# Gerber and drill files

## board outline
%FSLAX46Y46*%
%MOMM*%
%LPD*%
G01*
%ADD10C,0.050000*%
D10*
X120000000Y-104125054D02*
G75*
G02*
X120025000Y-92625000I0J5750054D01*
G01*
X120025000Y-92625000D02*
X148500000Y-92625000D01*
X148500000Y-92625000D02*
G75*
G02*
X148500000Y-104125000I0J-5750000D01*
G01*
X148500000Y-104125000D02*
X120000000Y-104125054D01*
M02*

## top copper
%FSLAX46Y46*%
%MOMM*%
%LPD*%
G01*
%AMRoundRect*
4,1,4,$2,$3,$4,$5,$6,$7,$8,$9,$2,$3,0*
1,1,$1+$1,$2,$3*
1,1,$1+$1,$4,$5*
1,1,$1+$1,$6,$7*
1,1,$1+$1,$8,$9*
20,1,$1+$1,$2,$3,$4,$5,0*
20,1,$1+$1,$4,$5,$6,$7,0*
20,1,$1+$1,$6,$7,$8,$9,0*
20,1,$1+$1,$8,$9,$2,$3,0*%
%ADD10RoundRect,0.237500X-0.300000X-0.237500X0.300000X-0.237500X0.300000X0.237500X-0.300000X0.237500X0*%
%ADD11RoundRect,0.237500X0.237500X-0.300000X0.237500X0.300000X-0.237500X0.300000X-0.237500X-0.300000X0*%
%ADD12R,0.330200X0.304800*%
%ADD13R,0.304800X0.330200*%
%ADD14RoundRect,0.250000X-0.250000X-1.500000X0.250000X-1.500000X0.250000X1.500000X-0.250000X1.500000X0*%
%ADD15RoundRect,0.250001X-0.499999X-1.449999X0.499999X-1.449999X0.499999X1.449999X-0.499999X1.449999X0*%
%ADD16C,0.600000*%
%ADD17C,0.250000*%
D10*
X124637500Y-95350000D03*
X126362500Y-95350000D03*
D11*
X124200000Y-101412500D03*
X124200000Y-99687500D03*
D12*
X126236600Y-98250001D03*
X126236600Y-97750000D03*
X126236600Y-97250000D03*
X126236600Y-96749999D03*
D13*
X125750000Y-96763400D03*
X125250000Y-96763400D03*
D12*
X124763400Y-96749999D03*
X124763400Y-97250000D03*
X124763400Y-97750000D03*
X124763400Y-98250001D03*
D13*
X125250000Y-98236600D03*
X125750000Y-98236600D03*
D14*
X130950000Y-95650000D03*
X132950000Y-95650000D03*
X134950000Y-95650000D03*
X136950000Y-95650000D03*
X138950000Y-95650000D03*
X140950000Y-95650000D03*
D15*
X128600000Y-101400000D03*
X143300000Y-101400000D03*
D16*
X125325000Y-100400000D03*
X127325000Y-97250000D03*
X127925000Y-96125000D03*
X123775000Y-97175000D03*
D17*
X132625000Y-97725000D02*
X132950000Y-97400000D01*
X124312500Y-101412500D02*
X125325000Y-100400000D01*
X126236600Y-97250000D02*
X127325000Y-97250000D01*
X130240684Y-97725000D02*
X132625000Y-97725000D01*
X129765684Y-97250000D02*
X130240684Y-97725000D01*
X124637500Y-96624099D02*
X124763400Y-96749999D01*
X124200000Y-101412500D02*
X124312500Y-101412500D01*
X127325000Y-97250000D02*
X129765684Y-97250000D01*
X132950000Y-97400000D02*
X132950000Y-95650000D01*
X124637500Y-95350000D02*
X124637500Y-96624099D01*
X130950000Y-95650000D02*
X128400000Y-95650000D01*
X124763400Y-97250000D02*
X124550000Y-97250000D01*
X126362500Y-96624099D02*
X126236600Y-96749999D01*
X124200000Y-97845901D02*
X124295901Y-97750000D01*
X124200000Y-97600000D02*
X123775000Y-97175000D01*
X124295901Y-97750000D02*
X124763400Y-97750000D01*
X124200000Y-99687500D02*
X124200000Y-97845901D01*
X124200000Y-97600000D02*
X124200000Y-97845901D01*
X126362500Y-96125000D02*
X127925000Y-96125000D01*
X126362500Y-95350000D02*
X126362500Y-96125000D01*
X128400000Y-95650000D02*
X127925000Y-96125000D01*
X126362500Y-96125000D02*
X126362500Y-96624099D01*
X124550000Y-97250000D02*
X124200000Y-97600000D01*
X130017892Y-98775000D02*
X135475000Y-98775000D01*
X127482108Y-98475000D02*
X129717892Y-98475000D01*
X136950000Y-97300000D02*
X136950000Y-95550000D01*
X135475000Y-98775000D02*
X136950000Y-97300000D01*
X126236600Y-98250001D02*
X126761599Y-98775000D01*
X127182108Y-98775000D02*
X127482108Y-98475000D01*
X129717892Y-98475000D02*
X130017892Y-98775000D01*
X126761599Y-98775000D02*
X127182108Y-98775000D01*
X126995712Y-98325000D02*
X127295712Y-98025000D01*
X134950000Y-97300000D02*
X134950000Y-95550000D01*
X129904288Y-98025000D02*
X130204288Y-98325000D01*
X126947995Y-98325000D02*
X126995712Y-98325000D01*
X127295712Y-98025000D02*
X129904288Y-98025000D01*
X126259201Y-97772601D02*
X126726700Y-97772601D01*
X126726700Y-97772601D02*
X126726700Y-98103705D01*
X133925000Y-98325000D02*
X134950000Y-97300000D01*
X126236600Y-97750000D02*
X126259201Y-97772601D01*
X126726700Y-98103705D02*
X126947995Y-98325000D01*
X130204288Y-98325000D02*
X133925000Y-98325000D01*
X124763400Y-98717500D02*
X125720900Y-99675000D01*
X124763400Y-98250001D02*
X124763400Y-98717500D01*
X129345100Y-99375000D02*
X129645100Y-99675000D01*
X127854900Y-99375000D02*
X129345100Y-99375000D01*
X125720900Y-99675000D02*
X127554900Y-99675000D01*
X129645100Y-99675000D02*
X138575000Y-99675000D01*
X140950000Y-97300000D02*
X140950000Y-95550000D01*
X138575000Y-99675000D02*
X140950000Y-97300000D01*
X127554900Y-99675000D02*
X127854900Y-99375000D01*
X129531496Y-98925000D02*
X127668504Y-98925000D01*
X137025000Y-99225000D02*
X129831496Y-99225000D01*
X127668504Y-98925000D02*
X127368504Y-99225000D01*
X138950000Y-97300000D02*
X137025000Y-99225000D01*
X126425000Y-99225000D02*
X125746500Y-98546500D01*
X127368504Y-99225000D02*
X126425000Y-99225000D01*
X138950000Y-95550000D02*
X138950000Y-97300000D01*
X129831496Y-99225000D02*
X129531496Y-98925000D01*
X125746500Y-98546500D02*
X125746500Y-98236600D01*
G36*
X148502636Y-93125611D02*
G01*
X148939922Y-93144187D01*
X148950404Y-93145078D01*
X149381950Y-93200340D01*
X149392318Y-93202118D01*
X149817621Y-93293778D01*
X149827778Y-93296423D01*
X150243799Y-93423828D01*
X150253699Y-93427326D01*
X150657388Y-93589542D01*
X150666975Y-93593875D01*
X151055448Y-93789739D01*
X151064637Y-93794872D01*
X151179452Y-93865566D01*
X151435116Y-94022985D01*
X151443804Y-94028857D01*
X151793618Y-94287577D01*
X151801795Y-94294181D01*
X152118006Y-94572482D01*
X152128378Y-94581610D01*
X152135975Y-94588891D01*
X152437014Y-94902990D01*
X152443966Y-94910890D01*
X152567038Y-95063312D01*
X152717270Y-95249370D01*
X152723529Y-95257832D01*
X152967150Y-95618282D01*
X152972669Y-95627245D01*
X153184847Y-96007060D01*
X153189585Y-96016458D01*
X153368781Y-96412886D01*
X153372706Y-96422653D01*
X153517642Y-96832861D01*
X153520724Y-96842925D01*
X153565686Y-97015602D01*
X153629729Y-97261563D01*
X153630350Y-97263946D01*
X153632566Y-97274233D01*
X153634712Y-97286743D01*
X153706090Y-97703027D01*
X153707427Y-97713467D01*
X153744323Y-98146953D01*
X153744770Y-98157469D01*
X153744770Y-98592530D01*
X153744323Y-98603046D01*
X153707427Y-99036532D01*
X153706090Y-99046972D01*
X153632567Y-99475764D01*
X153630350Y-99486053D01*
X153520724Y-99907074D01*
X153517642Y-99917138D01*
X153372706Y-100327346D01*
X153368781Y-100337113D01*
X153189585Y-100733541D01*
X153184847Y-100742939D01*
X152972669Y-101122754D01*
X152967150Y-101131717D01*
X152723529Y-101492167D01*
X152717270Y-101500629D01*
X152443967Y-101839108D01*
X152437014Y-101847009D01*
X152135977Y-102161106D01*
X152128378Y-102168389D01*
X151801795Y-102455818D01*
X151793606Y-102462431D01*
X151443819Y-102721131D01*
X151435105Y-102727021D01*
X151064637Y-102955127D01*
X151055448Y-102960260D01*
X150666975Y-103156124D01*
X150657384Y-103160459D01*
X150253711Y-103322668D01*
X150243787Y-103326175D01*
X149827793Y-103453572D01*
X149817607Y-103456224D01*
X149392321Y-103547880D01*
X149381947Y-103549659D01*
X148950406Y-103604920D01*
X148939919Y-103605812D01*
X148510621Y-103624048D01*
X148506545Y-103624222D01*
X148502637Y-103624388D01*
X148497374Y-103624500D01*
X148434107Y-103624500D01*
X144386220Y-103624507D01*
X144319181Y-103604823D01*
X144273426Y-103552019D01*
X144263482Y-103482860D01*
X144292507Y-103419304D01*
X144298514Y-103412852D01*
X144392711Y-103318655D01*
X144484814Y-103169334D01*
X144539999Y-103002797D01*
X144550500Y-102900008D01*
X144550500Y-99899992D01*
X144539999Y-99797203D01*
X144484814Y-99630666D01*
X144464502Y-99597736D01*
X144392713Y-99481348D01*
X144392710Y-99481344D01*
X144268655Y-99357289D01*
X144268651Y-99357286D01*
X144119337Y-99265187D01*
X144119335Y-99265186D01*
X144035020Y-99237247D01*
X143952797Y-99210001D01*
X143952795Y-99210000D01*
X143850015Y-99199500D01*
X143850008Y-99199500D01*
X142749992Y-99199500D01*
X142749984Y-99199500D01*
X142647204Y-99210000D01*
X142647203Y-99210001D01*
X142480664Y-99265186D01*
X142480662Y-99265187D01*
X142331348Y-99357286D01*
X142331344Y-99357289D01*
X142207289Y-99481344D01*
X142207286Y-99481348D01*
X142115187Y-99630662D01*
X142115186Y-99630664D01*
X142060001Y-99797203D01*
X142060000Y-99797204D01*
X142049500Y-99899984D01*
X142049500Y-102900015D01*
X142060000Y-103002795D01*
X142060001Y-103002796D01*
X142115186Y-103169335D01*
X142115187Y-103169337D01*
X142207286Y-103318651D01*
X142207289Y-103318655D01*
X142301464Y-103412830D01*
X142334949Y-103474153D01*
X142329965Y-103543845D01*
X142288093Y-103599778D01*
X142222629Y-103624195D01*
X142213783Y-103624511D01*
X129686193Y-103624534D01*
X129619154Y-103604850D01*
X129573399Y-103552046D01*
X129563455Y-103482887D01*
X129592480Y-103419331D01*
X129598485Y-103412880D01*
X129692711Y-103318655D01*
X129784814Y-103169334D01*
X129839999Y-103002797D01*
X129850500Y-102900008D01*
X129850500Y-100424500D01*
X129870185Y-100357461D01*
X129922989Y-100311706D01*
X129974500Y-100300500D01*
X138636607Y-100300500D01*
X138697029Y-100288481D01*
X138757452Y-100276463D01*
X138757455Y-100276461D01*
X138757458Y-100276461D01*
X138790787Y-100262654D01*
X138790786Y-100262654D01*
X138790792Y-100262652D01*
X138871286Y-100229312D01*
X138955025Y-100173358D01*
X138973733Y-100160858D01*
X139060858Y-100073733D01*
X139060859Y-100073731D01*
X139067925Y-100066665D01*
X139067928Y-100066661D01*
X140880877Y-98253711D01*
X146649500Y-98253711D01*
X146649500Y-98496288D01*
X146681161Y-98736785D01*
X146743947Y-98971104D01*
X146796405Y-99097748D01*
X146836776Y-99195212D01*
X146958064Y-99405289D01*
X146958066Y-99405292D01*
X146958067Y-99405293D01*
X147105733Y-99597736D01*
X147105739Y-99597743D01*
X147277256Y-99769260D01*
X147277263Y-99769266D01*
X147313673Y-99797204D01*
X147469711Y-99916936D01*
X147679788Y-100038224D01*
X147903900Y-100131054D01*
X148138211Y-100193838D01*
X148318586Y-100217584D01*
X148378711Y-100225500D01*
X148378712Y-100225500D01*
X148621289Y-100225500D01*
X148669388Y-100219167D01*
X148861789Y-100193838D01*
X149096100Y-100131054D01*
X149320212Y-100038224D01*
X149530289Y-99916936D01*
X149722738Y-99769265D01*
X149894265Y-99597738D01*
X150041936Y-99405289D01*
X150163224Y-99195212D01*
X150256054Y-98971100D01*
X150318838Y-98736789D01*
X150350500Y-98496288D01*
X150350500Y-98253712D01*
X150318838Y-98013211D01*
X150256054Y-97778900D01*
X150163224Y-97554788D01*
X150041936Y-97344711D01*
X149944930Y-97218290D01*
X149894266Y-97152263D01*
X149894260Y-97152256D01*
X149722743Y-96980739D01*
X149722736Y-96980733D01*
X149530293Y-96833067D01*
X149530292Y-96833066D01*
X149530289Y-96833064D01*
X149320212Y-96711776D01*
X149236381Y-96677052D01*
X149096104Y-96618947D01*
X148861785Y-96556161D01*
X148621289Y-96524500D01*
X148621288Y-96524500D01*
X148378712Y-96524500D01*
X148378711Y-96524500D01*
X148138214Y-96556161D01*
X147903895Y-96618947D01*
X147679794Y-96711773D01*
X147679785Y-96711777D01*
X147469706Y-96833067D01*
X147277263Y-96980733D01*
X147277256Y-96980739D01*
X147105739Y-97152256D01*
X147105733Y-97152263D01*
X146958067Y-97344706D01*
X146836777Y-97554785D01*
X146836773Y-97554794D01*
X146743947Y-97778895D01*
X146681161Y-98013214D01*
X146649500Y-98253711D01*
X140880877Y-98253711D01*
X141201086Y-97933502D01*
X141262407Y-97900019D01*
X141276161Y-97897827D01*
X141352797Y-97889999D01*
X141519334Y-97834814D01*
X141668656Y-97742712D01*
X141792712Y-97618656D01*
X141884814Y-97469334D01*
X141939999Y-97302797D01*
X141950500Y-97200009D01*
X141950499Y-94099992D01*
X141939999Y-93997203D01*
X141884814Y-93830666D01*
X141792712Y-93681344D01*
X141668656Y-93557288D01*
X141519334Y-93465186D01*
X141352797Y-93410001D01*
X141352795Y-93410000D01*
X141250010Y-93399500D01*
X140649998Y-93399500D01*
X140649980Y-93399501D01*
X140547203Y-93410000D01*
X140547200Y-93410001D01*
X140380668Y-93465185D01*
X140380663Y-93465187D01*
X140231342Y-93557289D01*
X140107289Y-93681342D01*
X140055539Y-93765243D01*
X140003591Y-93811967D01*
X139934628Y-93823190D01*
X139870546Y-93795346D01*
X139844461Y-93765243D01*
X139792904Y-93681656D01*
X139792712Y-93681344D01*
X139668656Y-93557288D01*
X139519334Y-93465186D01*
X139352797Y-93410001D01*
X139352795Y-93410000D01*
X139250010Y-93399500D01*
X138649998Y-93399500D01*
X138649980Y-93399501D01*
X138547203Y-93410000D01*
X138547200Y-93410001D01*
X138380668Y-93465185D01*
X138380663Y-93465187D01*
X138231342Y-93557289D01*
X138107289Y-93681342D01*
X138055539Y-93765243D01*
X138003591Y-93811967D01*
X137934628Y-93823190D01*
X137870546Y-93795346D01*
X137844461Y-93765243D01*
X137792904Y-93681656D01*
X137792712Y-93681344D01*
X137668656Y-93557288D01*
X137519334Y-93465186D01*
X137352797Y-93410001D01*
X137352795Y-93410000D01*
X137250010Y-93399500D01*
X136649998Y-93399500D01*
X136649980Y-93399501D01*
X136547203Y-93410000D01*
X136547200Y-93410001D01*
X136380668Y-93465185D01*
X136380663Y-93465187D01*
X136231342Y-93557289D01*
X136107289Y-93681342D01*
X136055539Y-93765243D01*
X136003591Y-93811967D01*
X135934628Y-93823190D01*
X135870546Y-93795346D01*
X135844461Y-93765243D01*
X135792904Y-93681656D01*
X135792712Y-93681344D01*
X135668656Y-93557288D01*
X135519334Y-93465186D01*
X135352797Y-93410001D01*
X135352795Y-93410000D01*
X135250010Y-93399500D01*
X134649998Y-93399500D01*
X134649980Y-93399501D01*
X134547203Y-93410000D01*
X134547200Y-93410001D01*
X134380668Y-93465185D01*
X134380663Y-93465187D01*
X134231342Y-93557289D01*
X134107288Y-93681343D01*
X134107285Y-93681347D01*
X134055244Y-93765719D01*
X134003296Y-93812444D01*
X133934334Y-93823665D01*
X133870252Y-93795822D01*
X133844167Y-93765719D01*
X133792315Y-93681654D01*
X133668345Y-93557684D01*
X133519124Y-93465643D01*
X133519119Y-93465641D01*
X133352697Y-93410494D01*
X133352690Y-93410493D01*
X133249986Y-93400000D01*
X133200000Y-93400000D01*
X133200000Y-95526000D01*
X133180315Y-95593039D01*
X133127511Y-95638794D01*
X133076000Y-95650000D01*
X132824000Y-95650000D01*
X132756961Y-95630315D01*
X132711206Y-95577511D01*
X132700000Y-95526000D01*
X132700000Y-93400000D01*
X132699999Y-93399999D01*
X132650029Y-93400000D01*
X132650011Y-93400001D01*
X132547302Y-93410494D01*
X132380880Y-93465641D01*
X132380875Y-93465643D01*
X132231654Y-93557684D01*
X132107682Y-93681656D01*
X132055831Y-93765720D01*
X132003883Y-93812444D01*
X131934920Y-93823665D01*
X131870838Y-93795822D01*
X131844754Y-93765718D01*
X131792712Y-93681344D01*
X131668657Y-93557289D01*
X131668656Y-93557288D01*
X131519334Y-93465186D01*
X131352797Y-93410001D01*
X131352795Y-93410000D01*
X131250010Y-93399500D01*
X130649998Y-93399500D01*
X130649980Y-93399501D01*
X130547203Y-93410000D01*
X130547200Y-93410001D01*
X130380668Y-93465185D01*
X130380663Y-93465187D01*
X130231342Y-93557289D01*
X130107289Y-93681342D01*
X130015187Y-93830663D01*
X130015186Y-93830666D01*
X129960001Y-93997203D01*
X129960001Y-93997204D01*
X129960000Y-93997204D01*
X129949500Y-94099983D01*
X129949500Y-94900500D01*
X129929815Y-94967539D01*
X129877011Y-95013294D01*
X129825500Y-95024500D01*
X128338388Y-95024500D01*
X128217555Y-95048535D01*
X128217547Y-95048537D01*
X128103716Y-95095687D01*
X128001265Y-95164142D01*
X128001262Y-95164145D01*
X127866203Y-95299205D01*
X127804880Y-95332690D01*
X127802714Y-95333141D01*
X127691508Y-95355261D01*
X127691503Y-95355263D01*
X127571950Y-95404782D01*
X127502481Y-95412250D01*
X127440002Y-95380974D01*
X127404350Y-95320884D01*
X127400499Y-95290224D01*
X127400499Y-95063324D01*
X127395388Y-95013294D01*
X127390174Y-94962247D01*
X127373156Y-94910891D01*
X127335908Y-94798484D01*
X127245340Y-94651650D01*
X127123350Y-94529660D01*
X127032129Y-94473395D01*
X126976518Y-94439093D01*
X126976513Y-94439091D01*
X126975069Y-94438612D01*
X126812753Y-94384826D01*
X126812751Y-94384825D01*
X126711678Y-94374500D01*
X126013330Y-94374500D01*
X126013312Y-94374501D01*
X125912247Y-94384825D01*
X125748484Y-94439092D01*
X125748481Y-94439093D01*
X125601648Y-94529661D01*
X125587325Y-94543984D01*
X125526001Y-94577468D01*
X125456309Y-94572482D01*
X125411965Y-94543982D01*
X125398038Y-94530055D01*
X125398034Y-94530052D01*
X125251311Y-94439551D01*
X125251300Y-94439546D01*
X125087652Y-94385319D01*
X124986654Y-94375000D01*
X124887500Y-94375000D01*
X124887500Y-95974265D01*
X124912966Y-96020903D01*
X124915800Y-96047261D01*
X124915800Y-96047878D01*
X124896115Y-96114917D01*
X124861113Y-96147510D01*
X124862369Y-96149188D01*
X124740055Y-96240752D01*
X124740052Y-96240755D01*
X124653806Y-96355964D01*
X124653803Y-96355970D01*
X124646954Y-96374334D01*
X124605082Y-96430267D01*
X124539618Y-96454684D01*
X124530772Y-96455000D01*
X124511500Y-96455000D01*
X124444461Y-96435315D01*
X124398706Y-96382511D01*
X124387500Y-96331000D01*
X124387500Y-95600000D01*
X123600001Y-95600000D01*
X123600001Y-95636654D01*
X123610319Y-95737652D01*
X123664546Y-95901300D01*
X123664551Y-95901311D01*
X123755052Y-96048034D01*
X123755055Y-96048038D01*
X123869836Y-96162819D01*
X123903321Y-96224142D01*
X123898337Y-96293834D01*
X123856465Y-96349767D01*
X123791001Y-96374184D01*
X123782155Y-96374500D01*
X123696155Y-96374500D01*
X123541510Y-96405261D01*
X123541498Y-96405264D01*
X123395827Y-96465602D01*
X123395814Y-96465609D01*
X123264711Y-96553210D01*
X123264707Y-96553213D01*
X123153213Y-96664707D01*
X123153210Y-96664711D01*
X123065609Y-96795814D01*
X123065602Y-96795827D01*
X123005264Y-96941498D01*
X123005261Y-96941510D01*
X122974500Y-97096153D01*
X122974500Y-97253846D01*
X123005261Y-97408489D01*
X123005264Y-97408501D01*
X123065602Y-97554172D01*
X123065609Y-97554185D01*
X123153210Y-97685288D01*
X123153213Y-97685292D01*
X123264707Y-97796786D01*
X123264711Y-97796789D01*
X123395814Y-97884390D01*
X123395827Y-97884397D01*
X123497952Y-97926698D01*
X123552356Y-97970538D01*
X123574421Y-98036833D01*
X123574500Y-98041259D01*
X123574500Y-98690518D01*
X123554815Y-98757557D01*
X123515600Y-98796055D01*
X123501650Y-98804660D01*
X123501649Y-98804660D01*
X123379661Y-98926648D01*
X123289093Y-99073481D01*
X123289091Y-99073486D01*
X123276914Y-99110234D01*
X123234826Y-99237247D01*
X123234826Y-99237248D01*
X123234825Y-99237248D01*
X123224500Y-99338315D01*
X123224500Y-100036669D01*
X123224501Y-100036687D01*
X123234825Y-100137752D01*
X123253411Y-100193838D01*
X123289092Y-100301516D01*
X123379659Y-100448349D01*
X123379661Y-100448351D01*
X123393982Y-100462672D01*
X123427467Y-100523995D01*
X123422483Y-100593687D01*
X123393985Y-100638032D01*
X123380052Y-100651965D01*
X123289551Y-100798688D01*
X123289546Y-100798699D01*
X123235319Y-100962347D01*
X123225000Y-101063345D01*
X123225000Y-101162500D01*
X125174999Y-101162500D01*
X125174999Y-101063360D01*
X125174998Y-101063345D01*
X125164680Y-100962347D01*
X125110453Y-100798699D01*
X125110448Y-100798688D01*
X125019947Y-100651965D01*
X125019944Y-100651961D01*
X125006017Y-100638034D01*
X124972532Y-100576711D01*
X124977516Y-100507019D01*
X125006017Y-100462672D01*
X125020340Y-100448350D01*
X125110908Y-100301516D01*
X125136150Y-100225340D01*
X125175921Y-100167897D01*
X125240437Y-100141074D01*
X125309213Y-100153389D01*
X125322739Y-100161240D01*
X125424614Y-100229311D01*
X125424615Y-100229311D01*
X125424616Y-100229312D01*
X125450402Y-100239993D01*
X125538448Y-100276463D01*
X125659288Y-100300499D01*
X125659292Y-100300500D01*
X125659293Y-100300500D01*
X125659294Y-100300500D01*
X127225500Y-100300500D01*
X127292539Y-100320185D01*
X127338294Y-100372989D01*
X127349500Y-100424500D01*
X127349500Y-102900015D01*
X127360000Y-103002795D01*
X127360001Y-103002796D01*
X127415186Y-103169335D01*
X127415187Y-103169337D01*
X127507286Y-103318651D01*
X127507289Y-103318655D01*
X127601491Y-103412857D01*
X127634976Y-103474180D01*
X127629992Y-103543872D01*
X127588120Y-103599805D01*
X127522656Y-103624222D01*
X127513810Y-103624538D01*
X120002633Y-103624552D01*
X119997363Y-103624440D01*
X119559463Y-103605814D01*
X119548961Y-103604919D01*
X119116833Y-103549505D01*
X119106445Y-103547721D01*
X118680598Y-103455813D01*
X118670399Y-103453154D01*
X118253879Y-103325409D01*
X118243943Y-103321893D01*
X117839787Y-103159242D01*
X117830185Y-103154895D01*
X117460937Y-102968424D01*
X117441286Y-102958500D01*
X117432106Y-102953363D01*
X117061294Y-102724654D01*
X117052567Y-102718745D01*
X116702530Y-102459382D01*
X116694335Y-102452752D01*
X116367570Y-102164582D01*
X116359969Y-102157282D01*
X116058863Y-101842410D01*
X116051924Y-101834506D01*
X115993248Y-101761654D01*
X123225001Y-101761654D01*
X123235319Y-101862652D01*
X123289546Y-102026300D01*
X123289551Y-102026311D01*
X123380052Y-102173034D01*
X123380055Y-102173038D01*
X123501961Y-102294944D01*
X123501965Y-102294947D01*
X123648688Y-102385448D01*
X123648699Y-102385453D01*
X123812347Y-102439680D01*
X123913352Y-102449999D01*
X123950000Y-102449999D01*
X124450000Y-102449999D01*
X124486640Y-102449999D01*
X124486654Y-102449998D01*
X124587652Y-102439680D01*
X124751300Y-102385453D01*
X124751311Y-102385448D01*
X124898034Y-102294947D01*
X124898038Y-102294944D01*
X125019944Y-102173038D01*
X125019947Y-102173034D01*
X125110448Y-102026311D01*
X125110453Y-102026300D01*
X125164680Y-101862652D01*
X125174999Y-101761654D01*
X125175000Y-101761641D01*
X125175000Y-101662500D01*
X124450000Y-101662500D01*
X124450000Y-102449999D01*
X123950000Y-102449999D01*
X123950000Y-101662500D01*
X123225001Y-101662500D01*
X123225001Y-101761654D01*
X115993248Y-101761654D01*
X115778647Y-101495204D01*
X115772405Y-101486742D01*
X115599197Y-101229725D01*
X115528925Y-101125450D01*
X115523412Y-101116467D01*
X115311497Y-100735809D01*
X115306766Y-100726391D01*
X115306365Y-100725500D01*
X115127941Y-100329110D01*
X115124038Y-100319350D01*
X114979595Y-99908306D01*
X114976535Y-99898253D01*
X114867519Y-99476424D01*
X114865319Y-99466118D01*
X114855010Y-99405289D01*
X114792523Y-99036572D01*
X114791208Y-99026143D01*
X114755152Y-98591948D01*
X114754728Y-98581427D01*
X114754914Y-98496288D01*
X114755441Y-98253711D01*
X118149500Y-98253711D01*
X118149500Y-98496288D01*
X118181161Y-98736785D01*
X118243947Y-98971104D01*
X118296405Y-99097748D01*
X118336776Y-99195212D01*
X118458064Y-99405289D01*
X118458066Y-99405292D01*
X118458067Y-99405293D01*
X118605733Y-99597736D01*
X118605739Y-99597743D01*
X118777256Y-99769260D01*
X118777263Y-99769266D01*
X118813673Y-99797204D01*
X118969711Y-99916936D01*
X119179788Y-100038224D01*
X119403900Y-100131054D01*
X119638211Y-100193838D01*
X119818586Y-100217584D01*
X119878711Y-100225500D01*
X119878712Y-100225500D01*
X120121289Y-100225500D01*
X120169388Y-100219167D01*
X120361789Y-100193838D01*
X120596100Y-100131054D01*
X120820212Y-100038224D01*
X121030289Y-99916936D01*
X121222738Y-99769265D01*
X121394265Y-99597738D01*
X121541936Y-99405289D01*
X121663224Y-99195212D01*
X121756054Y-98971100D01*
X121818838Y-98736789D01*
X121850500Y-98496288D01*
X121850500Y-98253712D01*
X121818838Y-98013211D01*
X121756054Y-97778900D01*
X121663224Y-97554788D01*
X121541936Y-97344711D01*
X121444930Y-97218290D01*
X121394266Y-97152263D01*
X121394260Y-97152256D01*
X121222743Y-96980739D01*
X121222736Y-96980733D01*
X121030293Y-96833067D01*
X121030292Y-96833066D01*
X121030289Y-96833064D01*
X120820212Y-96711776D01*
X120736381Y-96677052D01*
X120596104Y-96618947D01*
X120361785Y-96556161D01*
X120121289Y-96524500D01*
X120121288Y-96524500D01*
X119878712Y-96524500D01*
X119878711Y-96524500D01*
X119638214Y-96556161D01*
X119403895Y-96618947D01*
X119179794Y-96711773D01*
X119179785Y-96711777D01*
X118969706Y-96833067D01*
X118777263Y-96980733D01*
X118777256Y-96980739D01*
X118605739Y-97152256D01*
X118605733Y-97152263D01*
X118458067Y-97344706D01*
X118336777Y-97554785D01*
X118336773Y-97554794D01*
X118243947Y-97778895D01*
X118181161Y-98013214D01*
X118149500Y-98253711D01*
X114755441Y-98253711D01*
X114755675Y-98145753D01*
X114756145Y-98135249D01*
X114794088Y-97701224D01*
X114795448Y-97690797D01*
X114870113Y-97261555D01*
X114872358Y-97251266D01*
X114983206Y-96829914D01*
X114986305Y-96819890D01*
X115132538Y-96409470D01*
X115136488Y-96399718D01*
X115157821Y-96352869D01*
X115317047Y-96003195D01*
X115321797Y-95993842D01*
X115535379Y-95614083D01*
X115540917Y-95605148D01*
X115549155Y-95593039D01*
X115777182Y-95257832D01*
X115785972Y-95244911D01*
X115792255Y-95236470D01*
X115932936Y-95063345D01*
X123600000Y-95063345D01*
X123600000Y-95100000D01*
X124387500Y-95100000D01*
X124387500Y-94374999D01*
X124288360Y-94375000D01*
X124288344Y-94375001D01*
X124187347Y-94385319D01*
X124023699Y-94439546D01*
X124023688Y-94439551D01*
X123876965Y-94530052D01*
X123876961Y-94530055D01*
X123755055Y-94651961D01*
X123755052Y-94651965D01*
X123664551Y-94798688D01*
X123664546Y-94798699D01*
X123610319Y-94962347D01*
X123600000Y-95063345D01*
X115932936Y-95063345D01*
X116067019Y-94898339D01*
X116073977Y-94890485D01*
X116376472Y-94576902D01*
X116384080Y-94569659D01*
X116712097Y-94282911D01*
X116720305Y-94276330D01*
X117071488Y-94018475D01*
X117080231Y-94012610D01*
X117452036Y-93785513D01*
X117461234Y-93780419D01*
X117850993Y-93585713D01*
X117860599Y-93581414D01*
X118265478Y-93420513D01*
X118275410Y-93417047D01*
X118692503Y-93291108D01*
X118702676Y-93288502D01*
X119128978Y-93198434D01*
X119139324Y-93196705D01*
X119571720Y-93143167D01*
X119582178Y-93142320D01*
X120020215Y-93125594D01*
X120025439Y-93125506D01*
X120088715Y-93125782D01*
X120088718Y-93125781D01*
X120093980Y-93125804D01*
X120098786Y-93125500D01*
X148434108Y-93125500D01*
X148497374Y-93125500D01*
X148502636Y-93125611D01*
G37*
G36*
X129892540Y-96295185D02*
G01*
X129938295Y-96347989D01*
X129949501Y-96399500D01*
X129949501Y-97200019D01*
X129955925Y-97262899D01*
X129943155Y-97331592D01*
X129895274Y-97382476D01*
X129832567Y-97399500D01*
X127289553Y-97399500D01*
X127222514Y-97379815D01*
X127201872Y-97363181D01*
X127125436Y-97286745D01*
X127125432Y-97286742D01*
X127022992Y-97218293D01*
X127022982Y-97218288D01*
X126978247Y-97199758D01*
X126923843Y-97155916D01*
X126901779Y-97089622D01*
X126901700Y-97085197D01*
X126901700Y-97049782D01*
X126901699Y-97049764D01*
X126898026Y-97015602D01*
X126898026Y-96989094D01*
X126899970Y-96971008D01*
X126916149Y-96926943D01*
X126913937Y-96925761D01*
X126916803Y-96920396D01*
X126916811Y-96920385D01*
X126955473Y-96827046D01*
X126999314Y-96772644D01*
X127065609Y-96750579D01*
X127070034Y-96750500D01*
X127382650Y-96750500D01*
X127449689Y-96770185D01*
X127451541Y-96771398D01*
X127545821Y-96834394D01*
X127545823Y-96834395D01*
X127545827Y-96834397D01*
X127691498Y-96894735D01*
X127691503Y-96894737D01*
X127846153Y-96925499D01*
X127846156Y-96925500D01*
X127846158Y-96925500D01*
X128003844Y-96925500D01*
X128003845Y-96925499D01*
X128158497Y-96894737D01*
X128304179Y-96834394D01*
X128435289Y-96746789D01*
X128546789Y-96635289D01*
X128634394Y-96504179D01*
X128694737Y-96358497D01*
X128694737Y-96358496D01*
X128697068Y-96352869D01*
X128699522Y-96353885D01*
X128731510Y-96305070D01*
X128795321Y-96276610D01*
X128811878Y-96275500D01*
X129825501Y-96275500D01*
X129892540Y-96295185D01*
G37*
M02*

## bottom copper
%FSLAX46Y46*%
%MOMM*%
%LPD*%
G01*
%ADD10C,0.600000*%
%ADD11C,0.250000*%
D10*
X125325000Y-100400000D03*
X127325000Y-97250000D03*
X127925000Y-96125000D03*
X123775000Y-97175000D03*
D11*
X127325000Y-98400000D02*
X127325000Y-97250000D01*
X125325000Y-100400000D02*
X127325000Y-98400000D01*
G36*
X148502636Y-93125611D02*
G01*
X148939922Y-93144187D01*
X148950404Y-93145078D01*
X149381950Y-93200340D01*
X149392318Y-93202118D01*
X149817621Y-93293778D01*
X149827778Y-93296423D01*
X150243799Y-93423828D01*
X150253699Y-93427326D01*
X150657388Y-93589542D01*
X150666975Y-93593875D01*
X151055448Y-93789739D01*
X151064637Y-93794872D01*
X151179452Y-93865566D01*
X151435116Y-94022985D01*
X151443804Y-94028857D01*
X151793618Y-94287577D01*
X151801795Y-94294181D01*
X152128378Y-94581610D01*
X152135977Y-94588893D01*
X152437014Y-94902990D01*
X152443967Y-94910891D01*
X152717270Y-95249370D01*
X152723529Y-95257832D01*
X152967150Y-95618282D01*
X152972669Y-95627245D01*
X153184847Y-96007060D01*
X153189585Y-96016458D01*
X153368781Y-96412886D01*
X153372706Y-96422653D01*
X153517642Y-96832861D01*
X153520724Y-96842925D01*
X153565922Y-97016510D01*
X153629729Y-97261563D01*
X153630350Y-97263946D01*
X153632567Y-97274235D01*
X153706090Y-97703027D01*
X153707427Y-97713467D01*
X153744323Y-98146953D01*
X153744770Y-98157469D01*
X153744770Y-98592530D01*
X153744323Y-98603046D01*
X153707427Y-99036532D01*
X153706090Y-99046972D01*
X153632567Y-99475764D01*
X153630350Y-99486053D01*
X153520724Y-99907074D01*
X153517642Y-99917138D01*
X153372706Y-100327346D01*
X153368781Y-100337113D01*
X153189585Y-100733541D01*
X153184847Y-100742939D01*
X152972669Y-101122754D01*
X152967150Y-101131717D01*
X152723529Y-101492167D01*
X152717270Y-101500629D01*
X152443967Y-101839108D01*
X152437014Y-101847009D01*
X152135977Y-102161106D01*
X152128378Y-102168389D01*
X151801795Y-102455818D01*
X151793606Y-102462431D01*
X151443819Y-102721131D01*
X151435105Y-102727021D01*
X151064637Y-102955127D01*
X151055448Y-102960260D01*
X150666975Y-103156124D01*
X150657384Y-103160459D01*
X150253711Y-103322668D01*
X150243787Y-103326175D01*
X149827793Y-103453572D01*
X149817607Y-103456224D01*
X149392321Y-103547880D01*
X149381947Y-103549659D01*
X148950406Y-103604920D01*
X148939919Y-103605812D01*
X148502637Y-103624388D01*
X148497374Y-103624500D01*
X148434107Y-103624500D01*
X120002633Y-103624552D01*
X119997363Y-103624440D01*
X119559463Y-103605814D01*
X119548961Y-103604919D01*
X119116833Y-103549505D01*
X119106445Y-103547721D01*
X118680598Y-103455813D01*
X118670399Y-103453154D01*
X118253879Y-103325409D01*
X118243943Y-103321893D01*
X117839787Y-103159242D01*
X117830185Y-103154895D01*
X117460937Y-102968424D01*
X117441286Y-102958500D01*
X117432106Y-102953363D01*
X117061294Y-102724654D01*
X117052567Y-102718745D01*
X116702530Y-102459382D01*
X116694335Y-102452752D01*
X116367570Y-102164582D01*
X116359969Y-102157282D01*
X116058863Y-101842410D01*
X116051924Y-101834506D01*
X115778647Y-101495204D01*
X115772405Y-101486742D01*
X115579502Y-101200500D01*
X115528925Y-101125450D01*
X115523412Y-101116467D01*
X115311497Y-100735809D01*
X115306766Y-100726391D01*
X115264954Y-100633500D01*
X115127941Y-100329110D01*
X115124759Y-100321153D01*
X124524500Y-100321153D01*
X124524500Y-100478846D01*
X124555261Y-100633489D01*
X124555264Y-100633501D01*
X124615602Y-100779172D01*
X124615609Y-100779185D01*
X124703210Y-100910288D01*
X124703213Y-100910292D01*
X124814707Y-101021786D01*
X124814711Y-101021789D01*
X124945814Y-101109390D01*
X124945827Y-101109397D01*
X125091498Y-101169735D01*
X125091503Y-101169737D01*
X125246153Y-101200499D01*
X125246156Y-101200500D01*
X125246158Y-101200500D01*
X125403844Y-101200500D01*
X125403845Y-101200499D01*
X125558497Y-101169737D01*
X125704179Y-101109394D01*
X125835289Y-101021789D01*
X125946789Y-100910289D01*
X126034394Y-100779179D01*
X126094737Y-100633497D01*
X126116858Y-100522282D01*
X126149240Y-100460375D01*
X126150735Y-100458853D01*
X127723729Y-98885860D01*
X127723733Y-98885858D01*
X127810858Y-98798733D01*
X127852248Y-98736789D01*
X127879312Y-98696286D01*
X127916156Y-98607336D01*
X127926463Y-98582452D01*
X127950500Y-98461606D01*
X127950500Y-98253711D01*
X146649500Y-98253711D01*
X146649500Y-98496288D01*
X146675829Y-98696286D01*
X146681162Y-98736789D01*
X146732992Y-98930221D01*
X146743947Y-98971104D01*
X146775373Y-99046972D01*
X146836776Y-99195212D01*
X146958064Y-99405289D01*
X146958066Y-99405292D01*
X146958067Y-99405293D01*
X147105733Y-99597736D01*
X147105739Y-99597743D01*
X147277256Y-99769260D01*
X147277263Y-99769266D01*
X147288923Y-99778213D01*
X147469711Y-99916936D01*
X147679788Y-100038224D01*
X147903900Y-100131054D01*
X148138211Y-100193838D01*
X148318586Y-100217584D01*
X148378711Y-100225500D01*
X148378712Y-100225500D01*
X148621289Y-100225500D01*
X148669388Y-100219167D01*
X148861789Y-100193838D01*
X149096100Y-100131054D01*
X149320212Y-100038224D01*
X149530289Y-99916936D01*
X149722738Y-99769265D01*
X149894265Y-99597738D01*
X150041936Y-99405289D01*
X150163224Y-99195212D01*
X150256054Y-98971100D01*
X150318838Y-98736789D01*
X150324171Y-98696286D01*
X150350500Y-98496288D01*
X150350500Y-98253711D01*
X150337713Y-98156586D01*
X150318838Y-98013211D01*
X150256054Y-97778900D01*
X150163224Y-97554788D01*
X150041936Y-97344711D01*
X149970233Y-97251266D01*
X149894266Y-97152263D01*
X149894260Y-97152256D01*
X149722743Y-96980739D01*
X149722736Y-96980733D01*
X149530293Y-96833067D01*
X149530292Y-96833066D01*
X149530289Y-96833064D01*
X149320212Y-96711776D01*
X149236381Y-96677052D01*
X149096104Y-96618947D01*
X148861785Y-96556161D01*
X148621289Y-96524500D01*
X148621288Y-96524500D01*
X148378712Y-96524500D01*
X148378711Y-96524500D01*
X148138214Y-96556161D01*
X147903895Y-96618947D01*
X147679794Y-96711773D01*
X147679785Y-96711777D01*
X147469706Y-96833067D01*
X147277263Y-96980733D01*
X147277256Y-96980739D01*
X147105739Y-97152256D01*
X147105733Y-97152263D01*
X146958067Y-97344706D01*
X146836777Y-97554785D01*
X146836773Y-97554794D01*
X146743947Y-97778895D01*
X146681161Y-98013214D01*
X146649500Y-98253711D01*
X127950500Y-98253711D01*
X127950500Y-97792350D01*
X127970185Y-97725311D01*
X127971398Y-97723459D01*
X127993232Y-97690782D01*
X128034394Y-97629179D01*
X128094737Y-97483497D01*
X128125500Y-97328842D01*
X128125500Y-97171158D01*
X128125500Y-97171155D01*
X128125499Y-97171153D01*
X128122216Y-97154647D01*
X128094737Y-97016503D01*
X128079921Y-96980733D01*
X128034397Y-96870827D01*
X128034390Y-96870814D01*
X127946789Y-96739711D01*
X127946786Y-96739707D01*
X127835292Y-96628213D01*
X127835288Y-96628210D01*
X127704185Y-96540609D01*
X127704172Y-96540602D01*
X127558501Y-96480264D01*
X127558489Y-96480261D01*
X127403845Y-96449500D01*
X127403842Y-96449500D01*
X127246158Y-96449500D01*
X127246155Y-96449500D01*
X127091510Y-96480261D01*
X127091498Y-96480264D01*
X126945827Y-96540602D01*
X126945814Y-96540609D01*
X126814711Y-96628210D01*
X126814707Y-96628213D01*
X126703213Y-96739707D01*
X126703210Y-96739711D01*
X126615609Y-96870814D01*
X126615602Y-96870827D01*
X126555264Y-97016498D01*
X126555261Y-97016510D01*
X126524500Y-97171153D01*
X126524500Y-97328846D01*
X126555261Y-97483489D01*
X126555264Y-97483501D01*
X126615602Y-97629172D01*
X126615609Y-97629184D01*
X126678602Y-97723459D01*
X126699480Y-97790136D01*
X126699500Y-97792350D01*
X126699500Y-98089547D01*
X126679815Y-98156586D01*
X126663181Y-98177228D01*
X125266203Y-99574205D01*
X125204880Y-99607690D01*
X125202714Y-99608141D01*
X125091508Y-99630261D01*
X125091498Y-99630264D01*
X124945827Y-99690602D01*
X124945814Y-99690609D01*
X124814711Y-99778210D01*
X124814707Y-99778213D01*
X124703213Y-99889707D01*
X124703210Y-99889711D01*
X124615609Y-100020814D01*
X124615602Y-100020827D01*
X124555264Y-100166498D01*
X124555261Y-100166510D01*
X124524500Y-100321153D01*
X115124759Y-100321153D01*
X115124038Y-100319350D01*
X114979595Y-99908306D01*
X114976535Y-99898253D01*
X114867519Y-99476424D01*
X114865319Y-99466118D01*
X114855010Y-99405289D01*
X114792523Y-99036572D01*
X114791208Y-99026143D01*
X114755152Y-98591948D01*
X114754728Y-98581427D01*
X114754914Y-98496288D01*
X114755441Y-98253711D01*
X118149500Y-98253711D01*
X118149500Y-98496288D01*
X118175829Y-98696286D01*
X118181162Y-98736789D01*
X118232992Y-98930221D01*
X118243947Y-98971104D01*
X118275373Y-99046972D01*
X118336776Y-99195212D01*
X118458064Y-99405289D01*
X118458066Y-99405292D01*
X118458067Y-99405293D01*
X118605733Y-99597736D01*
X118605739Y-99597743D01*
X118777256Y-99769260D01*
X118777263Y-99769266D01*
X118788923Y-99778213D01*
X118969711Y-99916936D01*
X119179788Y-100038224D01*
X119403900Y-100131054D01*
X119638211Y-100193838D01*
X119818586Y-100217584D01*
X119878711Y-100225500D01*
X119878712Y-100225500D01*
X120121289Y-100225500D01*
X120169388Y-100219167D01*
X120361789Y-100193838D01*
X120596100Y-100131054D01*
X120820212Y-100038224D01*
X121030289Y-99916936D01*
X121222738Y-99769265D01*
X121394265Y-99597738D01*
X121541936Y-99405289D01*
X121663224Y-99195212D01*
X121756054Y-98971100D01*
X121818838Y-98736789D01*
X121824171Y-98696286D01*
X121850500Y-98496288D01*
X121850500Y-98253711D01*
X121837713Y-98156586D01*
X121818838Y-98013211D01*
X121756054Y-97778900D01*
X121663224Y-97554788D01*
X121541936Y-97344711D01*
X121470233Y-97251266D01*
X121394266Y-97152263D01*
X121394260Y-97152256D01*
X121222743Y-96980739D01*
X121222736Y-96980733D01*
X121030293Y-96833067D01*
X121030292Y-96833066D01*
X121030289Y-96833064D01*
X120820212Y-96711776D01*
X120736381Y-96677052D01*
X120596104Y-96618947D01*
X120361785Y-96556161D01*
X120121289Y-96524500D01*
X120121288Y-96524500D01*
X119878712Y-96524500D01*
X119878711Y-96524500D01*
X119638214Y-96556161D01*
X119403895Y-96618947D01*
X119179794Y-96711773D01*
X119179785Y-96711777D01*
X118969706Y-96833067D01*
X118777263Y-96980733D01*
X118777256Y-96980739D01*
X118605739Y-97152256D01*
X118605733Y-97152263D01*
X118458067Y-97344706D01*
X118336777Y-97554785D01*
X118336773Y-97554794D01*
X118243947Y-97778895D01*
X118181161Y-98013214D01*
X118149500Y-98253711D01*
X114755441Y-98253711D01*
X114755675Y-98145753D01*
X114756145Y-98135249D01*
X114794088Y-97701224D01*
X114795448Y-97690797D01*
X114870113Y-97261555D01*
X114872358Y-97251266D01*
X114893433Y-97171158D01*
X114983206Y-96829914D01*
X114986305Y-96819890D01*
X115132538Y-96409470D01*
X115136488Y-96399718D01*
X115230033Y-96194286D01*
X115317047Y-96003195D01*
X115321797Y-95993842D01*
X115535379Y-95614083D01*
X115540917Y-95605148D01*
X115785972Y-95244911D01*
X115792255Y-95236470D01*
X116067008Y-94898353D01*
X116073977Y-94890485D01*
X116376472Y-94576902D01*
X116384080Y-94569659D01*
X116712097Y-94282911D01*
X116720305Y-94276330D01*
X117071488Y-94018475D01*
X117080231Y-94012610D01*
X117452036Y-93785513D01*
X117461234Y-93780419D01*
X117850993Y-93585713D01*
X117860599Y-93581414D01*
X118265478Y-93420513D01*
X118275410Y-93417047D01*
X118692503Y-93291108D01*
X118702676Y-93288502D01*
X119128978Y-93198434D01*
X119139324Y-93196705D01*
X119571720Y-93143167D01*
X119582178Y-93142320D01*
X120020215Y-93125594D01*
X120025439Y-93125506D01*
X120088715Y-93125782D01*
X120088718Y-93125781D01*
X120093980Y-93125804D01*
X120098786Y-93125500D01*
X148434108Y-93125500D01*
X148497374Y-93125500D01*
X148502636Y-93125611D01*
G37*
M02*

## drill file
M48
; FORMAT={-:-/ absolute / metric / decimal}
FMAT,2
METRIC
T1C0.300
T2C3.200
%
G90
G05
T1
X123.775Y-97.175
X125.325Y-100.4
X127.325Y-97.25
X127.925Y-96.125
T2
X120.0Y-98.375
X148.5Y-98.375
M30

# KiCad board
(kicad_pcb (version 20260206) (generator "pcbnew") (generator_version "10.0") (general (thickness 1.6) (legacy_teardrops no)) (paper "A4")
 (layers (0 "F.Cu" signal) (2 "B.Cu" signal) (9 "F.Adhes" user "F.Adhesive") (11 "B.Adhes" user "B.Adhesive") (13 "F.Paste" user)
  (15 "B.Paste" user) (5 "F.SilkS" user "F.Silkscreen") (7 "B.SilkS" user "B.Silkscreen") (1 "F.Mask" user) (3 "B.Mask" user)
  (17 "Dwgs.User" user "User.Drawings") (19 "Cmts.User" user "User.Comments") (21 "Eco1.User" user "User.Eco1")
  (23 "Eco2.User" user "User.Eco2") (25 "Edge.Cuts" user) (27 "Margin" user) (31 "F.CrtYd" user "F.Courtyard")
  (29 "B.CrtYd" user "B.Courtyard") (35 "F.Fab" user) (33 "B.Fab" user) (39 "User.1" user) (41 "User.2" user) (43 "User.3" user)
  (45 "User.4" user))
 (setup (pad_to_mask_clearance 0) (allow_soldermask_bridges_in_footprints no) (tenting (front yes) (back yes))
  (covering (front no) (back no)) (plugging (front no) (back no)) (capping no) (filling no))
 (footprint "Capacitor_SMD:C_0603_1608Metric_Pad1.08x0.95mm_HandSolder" (layer "F.Cu") (at 125.5 95.35)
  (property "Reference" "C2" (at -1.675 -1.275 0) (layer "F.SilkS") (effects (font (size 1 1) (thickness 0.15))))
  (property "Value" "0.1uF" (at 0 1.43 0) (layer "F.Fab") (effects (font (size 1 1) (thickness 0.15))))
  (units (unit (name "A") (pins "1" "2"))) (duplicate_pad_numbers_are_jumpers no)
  (pad "1" smd roundrect (at -0.8625 0) (size 1.075 0.95) (layers "F.Cu" "F.Mask" "F.Paste") (roundrect_rratio 0.25) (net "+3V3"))
  (pad "2" smd roundrect (at 0.8625 0) (size 1.075 0.95) (layers "F.Cu" "F.Mask" "F.Paste") (roundrect_rratio 0.25) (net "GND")))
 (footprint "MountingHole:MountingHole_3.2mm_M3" (layer "F.Cu") (at 148.5 98.375)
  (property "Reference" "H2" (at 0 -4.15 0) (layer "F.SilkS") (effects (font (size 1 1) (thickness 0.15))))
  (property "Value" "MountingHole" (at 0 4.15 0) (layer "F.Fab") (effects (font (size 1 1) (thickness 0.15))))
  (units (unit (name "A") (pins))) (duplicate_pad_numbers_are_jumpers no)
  (pad "" np_thru_hole circle (at 0 0) (size 3.2 3.2) (drill 3.2) (layers "*.Cu" "*.Mask")))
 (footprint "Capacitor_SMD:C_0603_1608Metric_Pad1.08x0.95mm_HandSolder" (layer "F.Cu") (at 124.2 100.55 90)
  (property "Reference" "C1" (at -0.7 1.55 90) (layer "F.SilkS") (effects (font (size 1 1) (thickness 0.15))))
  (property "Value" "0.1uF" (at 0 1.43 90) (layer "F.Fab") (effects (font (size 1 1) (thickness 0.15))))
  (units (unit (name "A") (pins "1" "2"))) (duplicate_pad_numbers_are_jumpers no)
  (pad "1" smd roundrect (at -0.8625 0 90) (size 1.075 0.95) (layers "F.Cu" "F.Mask" "F.Paste") (roundrect_rratio 0.25) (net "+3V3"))
  (pad "2" smd roundrect (at 0.8625 0 90) (size 1.075 0.95) (layers "F.Cu" "F.Mask" "F.Paste") (roundrect_rratio 0.25) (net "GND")))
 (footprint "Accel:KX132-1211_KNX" (layer "F.Cu") (at 125.5 97.5 180)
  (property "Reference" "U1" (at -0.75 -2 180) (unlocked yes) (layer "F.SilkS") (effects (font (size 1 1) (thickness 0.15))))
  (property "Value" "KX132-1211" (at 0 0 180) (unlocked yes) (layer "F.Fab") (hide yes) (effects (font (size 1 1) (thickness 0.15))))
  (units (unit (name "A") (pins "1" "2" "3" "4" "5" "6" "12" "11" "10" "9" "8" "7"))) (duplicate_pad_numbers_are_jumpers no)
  (pad "1" smd rect (at -0.7366 -0.750001 270) (size 0.3048 0.3302) (layers "F.Cu" "F.Mask" "F.Paste") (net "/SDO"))
  (pad "2" smd rect (at -0.7366 -0.25 270) (size 0.3048 0.3302) (layers "F.Cu" "F.Mask" "F.Paste") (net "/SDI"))
  (pad "3" smd rect (at -0.7366 0.25 270) (size 0.3048 0.3302) (layers "F.Cu" "F.Mask" "F.Paste") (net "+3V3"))
  (pad "4" smd rect (at -0.7366 0.750001 270) (size 0.3048 0.3302) (layers "F.Cu" "F.Mask" "F.Paste") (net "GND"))
  (pad "5" smd rect (at -0.25 0.7366 180) (size 0.3048 0.3302) (layers "F.Cu" "F.Mask" "F.Paste") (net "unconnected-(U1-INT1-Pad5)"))
  (pad "6" smd rect (at 0.25 0.7366 180) (size 0.3048 0.3302) (layers "F.Cu" "F.Mask" "F.Paste") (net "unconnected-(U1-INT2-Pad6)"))
  (pad "7" smd rect (at 0.7366 0.750001 270) (size 0.3048 0.3302) (layers "F.Cu" "F.Mask" "F.Paste") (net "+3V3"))
  (pad "8" smd rect (at 0.7366 0.25 270) (size 0.3048 0.3302) (layers "F.Cu" "F.Mask" "F.Paste") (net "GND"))
  (pad "9" smd rect (at 0.7366 -0.25 270) (size 0.3048 0.3302) (layers "F.Cu" "F.Mask" "F.Paste") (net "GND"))
  (pad "10" smd rect (at 0.7366 -0.750001 270) (size 0.3048 0.3302) (layers "F.Cu" "F.Mask" "F.Paste") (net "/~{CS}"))
  (pad "11" smd rect (at 0.25 -0.7366 180) (size 0.3048 0.3302) (layers "F.Cu" "F.Mask" "F.Paste") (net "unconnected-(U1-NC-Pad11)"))
  (pad "12" smd rect (at -0.25 -0.7366 180) (size 0.3048 0.3302) (layers "F.Cu" "F.Mask" "F.Paste") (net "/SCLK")))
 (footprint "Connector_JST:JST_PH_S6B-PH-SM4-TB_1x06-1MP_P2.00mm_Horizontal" (layer "F.Cu") (at 135.95 98.5)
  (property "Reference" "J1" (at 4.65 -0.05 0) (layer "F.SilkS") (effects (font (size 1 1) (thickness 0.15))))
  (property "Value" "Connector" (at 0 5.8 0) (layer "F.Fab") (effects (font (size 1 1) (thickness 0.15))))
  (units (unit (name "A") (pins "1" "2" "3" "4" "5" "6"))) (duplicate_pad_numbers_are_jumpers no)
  (pad "1" smd roundrect (at -5 -2.85) (size 1 3.5) (layers "F.Cu" "F.Mask" "F.Paste") (roundrect_rratio 0.25) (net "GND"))
  (pad "2" smd roundrect (at -3 -2.85) (size 1 3.5) (layers "F.Cu" "F.Mask" "F.Paste") (roundrect_rratio 0.25) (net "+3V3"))
  (pad "3" smd roundrect (at -1 -2.85) (size 1 3.5) (layers "F.Cu" "F.Mask" "F.Paste") (roundrect_rratio 0.25) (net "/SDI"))
  (pad "4" smd roundrect (at 1 -2.85) (size 1 3.5) (layers "F.Cu" "F.Mask" "F.Paste") (roundrect_rratio 0.25) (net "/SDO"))
  (pad "5" smd roundrect (at 3 -2.85) (size 1 3.5) (layers "F.Cu" "F.Mask" "F.Paste") (roundrect_rratio 0.25) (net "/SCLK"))
  (pad "6" smd roundrect (at 5 -2.85) (size 1 3.5) (layers "F.Cu" "F.Mask" "F.Paste") (roundrect_rratio 0.25) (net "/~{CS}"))
  (pad "MP" smd roundrect (at -7.35 2.9) (size 1.5 3.4) (layers "F.Cu" "F.Mask" "F.Paste") (roundrect_rratio 0.166667))
  (pad "MP" smd roundrect (at 7.35 2.9) (size 1.5 3.4) (layers "F.Cu" "F.Mask" "F.Paste") (roundrect_rratio 0.166667)))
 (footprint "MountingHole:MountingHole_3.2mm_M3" (layer "F.Cu") (at 120 98.375)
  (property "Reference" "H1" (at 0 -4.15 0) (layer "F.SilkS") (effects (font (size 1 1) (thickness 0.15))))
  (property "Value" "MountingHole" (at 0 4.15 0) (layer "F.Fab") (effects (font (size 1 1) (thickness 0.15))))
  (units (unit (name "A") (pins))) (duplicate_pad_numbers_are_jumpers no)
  (pad "" np_thru_hole circle (at 0 0) (size 3.2 3.2) (drill 3.2) (layers "*.Cu" "*.Mask")))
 (gr_arc (start 120 104.125054) (mid 114.24996 98.3625) (end 120.025 92.625) (stroke (width 0.05) (type default)) (layer "Edge.Cuts"))
 (gr_line (start 120.025 92.625) (end 148.5 92.625) (stroke (width 0.05) (type default)) (layer "Edge.Cuts"))
 (gr_arc (start 148.5 92.625) (mid 154.25 98.375) (end 148.5 104.125) (stroke (width 0.05) (type default)) (layer "Edge.Cuts"))
 (gr_line (start 148.5 104.125) (end 120 104.125054) (stroke (width 0.05) (type default)) (layer "Edge.Cuts"))
 (segment (start 132.625 97.725) (end 132.95 97.4) (width 0.25) (layer "F.Cu") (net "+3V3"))
 (segment (start 124.3125 101.4125) (end 125.325 100.4) (width 0.25) (layer "F.Cu") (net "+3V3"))
 (segment (start 126.2366 97.25) (end 127.325 97.25) (width 0.25) (layer "F.Cu") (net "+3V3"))
 (segment (start 130.240684 97.725) (end 132.625 97.725) (width 0.25) (layer "F.Cu") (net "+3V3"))
 (segment (start 129.765684 97.25) (end 130.240684 97.725) (width 0.25) (layer "F.Cu") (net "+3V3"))
 (segment (start 124.6375 96.624099) (end 124.7634 96.749999) (width 0.25) (layer "F.Cu") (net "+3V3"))
 (segment (start 124.2 101.4125) (end 124.3125 101.4125) (width 0.25) (layer "F.Cu") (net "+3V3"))
 (segment (start 127.325 97.25) (end 129.765684 97.25) (width 0.25) (layer "F.Cu") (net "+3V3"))
 (segment (start 132.95 97.4) (end 132.95 95.65) (width 0.25) (layer "F.Cu") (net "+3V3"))
 (segment (start 124.6375 95.35) (end 124.6375 96.624099) (width 0.25) (layer "F.Cu") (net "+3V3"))
 (via (at 125.325 100.4) (size 0.6) (drill 0.3) (layers "F.Cu" "B.Cu") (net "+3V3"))
 (via (at 127.325 97.25) (size 0.6) (drill 0.3) (layers "F.Cu" "B.Cu") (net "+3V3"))
 (segment (start 127.325 98.4) (end 127.325 97.25) (width 0.25) (layer "B.Cu") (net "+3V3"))
 (segment (start 125.325 100.4) (end 127.325 98.4) (width 0.25) (layer "B.Cu") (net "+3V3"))
 (segment (start 130.95 95.65) (end 128.4 95.65) (width 0.25) (layer "F.Cu") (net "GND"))
 (segment (start 124.7634 97.25) (end 124.55 97.25) (width 0.25) (layer "F.Cu") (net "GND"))
 (segment (start 126.3625 96.624099) (end 126.2366 96.749999) (width 0.25) (layer "F.Cu") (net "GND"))
 (segment (start 124.2 97.845901) (end 124.295901 97.75) (width 0.25) (layer "F.Cu") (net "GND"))
 (segment (start 124.2 97.6) (end 123.775 97.175) (width 0.25) (layer "F.Cu") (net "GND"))
 (segment (start 124.295901 97.75) (end 124.7634 97.75) (width 0.25) (layer "F.Cu") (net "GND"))
 (segment (start 124.2 99.6875) (end 124.2 97.845901) (width 0.25) (layer "F.Cu") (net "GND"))
 (segment (start 124.2 97.6) (end 124.2 97.845901) (width 0.25) (layer "F.Cu") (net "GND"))
 (segment (start 126.3625 96.125) (end 127.925 96.125) (width 0.25) (layer "F.Cu") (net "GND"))
 (segment (start 126.3625 95.35) (end 126.3625 96.125) (width 0.25) (layer "F.Cu") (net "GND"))
 (segment (start 128.4 95.65) (end 127.925 96.125) (width 0.25) (layer "F.Cu") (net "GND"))
 (segment (start 126.3625 96.125) (end 126.3625 96.624099) (width 0.25) (layer "F.Cu") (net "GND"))
 (segment (start 124.55 97.25) (end 124.2 97.6) (width 0.25) (layer "F.Cu") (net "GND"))
 (via (at 127.925 96.125) (size 0.6) (drill 0.3) (layers "F.Cu" "B.Cu") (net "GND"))
 (via (at 123.775 97.175) (size 0.6) (drill 0.3) (layers "F.Cu" "B.Cu") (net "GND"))
 (segment (start 130.017892 98.775) (end 135.475 98.775) (width 0.25) (layer "F.Cu") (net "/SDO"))
 (segment (start 127.482108 98.475) (end 129.717892 98.475) (width 0.25) (layer "F.Cu") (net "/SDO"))
 (segment (start 136.95 97.3) (end 136.95 95.55) (width 0.25) (layer "F.Cu") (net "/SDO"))
 (segment (start 135.475 98.775) (end 136.95 97.3) (width 0.25) (layer "F.Cu") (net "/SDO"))
 (segment (start 126.2366 98.250001) (end 126.761599 98.775) (width 0.25) (layer "F.Cu") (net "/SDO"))
 (segment (start 127.182108 98.775) (end 127.482108 98.475) (width 0.25) (layer "F.Cu") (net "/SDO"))
 (segment (start 129.717892 98.475) (end 130.017892 98.775) (width 0.25) (layer "F.Cu") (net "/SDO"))
 (segment (start 126.761599 98.775) (end 127.182108 98.775) (width 0.25) (layer "F.Cu") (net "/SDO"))
 (segment (start 126.995712 98.325) (end 127.295712 98.025) (width 0.25) (layer "F.Cu") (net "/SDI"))
 (segment (start 134.95 97.3) (end 134.95 95.55) (width 0.25) (layer "F.Cu") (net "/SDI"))
 (segment (start 129.904288 98.025) (end 130.204288 98.325) (width 0.25) (layer "F.Cu") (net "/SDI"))
 (segment (start 126.947995 98.325) (end 126.995712 98.325) (width 0.25) (layer "F.Cu") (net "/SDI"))
 (segment (start 127.295712 98.025) (end 129.904288 98.025) (width 0.25) (layer "F.Cu") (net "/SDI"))
 (segment (start 126.259201 97.772601) (end 126.7267 97.772601) (width 0.25) (layer "F.Cu") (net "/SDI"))
 (segment (start 126.7267 97.772601) (end 126.7267 98.103705) (width 0.25) (layer "F.Cu") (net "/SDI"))
 (segment (start 133.925 98.325) (end 134.95 97.3) (width 0.25) (layer "F.Cu") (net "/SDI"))
 (segment (start 126.2366 97.75) (end 126.259201 97.772601) (width 0.25) (layer "F.Cu") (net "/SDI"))
 (segment (start 126.7267 98.103705) (end 126.947995 98.325) (width 0.25) (layer "F.Cu") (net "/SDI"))
 (segment (start 130.204288 98.325) (end 133.925 98.325) (width 0.25) (layer "F.Cu") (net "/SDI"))
 (segment (start 124.7634 98.7175) (end 125.7209 99.675) (width 0.25) (layer "F.Cu") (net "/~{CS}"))
 (segment (start 124.7634 98.250001) (end 124.7634 98.7175) (width 0.25) (layer "F.Cu") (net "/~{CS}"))
 (segment (start 129.3451 99.375) (end 129.6451 99.675) (width 0.25) (layer "F.Cu") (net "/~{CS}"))
 (segment (start 127.8549 99.375) (end 129.3451 99.375) (width 0.25) (layer "F.Cu") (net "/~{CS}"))
 (segment (start 125.7209 99.675) (end 127.5549 99.675) (width 0.25) (layer "F.Cu") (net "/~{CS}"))
 (segment (start 129.6451 99.675) (end 138.575 99.675) (width 0.25) (layer "F.Cu") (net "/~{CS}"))
 (segment (start 140.95 97.3) (end 140.95 95.55) (width 0.25) (layer "F.Cu") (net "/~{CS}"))
 (segment (start 138.575 99.675) (end 140.95 97.3) (width 0.25) (layer "F.Cu") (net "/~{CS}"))
 (segment (start 127.5549 99.675) (end 127.8549 99.375) (width 0.25) (layer "F.Cu") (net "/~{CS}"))
 (segment (start 129.531496 98.925) (end 127.668504 98.925) (width 0.25) (layer "F.Cu") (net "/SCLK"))
 (segment (start 137.025 99.225) (end 129.831496 99.225) (width 0.25) (layer "F.Cu") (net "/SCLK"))
 (segment (start 127.668504 98.925) (end 127.368504 99.225) (width 0.25) (layer "F.Cu") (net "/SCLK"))
 (segment (start 138.95 97.3) (end 137.025 99.225) (width 0.25) (layer "F.Cu") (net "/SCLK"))
 (segment (start 126.425 99.225) (end 125.7465 98.5465) (width 0.25) (layer "F.Cu") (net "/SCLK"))
 (segment (start 127.368504 99.225) (end 126.425 99.225) (width 0.25) (layer "F.Cu") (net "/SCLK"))
 (segment (start 138.95 95.55) (end 138.95 97.3) (width 0.25) (layer "F.Cu") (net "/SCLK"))
 (segment (start 129.831496 99.225) (end 129.531496 98.925) (width 0.25) (layer "F.Cu") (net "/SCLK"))
 (segment (start 125.7465 98.5465) (end 125.7465 98.2366) (width 0.25) (layer "F.Cu") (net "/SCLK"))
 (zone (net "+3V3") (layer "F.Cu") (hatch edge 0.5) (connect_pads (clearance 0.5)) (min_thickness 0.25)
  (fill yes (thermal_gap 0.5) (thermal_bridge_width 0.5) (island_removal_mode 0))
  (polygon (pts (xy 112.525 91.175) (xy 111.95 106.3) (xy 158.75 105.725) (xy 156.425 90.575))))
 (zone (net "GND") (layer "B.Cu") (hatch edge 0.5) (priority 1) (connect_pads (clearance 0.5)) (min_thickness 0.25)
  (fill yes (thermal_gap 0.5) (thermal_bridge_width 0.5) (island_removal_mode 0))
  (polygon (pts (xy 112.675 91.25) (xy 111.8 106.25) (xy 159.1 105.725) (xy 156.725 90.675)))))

